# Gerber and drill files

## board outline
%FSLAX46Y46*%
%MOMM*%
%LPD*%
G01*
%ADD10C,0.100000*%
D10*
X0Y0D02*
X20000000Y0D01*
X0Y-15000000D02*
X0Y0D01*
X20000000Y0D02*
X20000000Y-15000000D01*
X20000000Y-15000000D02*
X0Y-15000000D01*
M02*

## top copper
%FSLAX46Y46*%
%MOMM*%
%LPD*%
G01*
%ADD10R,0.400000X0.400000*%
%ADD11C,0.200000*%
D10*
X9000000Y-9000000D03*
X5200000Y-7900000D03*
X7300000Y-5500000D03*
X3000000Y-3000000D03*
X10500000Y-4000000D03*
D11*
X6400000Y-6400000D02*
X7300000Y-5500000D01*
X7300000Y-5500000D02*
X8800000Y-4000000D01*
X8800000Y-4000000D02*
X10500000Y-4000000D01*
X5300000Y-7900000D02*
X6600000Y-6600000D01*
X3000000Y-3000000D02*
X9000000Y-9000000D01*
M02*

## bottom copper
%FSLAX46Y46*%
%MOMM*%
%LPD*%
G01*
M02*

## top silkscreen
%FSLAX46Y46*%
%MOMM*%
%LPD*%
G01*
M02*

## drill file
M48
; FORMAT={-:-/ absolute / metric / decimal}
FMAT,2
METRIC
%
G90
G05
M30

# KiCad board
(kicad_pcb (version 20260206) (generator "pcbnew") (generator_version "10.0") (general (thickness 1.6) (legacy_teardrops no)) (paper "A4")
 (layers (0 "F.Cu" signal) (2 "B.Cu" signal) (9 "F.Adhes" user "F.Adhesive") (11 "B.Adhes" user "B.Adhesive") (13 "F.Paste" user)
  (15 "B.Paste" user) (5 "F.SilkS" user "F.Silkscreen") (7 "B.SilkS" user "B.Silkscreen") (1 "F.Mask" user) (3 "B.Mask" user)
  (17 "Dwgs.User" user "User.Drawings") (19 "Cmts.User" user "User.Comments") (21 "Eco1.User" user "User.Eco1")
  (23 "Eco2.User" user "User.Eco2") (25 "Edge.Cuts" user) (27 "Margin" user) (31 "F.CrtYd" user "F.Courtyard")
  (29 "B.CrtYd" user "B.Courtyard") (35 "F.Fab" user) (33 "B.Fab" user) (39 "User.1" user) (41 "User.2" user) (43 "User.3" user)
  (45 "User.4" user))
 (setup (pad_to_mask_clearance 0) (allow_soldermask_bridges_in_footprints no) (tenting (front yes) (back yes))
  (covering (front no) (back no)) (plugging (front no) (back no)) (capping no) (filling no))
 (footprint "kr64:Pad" (layer "F.Cu") (at 9 9)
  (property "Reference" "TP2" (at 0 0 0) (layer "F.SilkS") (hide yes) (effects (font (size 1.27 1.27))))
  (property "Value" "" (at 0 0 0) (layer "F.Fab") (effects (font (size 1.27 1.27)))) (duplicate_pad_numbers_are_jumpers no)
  (pad "1" smd rect (at 0 0) (size 0.4 0.4) (layers "F.Cu" "F.Mask" "F.Paste") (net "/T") (thermal_bridge_angle 45)))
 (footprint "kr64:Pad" (layer "F.Cu") (at 5.2 7.9)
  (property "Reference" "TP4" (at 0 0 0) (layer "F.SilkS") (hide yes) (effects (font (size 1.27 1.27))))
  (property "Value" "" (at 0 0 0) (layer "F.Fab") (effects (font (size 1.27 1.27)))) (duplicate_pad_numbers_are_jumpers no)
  (pad "1" smd rect (at 0 0) (size 0.4 0.4) (layers "F.Cu" "F.Mask" "F.Paste") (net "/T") (thermal_bridge_angle 45)))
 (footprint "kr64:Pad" (layer "F.Cu") (at 7.3 5.5)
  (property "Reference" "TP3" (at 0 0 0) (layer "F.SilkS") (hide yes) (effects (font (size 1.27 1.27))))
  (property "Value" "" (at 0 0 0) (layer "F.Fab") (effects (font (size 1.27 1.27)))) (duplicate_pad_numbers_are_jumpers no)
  (pad "1" smd rect (at 0 0) (size 0.4 0.4) (layers "F.Cu" "F.Mask" "F.Paste") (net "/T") (thermal_bridge_angle 45)))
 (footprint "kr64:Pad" (layer "F.Cu") (at 3 3)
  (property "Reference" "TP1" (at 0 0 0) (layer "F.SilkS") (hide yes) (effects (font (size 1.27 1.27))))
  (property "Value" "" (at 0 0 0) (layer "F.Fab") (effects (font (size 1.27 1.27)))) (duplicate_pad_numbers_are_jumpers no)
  (pad "1" smd rect (at 0 0) (size 0.4 0.4) (layers "F.Cu" "F.Mask" "F.Paste") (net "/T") (thermal_bridge_angle 45)))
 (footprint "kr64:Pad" (layer "F.Cu") (at 10.5 4)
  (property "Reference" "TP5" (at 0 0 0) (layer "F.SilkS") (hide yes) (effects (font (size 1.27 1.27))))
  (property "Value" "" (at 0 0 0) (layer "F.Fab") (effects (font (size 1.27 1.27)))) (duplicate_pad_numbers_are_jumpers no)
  (pad "1" smd rect (at 0 0) (size 0.4 0.4) (layers "F.Cu" "F.Mask" "F.Paste") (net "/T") (thermal_bridge_angle 45)))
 (gr_line (start 0 0) (end 20 0) (stroke (width 0.1) (type default)) (layer "Edge.Cuts"))
 (gr_line (start 0 15) (end 0 0) (stroke (width 0.1) (type default)) (layer "Edge.Cuts"))
 (gr_line (start 20 0) (end 20 15) (stroke (width 0.1) (type default)) (layer "Edge.Cuts"))
 (gr_line (start 20 15) (end 0 15) (stroke (width 0.1) (type default)) (layer "Edge.Cuts"))
 (segment (start 6.4 6.4) (end 7.3 5.5) (width 0.2) (layer "F.Cu") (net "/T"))
 (segment (start 7.3 5.5) (end 8.8 4) (width 0.2) (layer "F.Cu") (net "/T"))
 (segment (start 8.8 4) (end 10.5 4) (width 0.2) (layer "F.Cu") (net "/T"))
 (segment (start 5.3 7.9) (end 6.6 6.6) (width 0.2) (layer "F.Cu") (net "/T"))
 (segment (start 3 3) (end 9 9) (width 0.2) (layer "F.Cu") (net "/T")))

